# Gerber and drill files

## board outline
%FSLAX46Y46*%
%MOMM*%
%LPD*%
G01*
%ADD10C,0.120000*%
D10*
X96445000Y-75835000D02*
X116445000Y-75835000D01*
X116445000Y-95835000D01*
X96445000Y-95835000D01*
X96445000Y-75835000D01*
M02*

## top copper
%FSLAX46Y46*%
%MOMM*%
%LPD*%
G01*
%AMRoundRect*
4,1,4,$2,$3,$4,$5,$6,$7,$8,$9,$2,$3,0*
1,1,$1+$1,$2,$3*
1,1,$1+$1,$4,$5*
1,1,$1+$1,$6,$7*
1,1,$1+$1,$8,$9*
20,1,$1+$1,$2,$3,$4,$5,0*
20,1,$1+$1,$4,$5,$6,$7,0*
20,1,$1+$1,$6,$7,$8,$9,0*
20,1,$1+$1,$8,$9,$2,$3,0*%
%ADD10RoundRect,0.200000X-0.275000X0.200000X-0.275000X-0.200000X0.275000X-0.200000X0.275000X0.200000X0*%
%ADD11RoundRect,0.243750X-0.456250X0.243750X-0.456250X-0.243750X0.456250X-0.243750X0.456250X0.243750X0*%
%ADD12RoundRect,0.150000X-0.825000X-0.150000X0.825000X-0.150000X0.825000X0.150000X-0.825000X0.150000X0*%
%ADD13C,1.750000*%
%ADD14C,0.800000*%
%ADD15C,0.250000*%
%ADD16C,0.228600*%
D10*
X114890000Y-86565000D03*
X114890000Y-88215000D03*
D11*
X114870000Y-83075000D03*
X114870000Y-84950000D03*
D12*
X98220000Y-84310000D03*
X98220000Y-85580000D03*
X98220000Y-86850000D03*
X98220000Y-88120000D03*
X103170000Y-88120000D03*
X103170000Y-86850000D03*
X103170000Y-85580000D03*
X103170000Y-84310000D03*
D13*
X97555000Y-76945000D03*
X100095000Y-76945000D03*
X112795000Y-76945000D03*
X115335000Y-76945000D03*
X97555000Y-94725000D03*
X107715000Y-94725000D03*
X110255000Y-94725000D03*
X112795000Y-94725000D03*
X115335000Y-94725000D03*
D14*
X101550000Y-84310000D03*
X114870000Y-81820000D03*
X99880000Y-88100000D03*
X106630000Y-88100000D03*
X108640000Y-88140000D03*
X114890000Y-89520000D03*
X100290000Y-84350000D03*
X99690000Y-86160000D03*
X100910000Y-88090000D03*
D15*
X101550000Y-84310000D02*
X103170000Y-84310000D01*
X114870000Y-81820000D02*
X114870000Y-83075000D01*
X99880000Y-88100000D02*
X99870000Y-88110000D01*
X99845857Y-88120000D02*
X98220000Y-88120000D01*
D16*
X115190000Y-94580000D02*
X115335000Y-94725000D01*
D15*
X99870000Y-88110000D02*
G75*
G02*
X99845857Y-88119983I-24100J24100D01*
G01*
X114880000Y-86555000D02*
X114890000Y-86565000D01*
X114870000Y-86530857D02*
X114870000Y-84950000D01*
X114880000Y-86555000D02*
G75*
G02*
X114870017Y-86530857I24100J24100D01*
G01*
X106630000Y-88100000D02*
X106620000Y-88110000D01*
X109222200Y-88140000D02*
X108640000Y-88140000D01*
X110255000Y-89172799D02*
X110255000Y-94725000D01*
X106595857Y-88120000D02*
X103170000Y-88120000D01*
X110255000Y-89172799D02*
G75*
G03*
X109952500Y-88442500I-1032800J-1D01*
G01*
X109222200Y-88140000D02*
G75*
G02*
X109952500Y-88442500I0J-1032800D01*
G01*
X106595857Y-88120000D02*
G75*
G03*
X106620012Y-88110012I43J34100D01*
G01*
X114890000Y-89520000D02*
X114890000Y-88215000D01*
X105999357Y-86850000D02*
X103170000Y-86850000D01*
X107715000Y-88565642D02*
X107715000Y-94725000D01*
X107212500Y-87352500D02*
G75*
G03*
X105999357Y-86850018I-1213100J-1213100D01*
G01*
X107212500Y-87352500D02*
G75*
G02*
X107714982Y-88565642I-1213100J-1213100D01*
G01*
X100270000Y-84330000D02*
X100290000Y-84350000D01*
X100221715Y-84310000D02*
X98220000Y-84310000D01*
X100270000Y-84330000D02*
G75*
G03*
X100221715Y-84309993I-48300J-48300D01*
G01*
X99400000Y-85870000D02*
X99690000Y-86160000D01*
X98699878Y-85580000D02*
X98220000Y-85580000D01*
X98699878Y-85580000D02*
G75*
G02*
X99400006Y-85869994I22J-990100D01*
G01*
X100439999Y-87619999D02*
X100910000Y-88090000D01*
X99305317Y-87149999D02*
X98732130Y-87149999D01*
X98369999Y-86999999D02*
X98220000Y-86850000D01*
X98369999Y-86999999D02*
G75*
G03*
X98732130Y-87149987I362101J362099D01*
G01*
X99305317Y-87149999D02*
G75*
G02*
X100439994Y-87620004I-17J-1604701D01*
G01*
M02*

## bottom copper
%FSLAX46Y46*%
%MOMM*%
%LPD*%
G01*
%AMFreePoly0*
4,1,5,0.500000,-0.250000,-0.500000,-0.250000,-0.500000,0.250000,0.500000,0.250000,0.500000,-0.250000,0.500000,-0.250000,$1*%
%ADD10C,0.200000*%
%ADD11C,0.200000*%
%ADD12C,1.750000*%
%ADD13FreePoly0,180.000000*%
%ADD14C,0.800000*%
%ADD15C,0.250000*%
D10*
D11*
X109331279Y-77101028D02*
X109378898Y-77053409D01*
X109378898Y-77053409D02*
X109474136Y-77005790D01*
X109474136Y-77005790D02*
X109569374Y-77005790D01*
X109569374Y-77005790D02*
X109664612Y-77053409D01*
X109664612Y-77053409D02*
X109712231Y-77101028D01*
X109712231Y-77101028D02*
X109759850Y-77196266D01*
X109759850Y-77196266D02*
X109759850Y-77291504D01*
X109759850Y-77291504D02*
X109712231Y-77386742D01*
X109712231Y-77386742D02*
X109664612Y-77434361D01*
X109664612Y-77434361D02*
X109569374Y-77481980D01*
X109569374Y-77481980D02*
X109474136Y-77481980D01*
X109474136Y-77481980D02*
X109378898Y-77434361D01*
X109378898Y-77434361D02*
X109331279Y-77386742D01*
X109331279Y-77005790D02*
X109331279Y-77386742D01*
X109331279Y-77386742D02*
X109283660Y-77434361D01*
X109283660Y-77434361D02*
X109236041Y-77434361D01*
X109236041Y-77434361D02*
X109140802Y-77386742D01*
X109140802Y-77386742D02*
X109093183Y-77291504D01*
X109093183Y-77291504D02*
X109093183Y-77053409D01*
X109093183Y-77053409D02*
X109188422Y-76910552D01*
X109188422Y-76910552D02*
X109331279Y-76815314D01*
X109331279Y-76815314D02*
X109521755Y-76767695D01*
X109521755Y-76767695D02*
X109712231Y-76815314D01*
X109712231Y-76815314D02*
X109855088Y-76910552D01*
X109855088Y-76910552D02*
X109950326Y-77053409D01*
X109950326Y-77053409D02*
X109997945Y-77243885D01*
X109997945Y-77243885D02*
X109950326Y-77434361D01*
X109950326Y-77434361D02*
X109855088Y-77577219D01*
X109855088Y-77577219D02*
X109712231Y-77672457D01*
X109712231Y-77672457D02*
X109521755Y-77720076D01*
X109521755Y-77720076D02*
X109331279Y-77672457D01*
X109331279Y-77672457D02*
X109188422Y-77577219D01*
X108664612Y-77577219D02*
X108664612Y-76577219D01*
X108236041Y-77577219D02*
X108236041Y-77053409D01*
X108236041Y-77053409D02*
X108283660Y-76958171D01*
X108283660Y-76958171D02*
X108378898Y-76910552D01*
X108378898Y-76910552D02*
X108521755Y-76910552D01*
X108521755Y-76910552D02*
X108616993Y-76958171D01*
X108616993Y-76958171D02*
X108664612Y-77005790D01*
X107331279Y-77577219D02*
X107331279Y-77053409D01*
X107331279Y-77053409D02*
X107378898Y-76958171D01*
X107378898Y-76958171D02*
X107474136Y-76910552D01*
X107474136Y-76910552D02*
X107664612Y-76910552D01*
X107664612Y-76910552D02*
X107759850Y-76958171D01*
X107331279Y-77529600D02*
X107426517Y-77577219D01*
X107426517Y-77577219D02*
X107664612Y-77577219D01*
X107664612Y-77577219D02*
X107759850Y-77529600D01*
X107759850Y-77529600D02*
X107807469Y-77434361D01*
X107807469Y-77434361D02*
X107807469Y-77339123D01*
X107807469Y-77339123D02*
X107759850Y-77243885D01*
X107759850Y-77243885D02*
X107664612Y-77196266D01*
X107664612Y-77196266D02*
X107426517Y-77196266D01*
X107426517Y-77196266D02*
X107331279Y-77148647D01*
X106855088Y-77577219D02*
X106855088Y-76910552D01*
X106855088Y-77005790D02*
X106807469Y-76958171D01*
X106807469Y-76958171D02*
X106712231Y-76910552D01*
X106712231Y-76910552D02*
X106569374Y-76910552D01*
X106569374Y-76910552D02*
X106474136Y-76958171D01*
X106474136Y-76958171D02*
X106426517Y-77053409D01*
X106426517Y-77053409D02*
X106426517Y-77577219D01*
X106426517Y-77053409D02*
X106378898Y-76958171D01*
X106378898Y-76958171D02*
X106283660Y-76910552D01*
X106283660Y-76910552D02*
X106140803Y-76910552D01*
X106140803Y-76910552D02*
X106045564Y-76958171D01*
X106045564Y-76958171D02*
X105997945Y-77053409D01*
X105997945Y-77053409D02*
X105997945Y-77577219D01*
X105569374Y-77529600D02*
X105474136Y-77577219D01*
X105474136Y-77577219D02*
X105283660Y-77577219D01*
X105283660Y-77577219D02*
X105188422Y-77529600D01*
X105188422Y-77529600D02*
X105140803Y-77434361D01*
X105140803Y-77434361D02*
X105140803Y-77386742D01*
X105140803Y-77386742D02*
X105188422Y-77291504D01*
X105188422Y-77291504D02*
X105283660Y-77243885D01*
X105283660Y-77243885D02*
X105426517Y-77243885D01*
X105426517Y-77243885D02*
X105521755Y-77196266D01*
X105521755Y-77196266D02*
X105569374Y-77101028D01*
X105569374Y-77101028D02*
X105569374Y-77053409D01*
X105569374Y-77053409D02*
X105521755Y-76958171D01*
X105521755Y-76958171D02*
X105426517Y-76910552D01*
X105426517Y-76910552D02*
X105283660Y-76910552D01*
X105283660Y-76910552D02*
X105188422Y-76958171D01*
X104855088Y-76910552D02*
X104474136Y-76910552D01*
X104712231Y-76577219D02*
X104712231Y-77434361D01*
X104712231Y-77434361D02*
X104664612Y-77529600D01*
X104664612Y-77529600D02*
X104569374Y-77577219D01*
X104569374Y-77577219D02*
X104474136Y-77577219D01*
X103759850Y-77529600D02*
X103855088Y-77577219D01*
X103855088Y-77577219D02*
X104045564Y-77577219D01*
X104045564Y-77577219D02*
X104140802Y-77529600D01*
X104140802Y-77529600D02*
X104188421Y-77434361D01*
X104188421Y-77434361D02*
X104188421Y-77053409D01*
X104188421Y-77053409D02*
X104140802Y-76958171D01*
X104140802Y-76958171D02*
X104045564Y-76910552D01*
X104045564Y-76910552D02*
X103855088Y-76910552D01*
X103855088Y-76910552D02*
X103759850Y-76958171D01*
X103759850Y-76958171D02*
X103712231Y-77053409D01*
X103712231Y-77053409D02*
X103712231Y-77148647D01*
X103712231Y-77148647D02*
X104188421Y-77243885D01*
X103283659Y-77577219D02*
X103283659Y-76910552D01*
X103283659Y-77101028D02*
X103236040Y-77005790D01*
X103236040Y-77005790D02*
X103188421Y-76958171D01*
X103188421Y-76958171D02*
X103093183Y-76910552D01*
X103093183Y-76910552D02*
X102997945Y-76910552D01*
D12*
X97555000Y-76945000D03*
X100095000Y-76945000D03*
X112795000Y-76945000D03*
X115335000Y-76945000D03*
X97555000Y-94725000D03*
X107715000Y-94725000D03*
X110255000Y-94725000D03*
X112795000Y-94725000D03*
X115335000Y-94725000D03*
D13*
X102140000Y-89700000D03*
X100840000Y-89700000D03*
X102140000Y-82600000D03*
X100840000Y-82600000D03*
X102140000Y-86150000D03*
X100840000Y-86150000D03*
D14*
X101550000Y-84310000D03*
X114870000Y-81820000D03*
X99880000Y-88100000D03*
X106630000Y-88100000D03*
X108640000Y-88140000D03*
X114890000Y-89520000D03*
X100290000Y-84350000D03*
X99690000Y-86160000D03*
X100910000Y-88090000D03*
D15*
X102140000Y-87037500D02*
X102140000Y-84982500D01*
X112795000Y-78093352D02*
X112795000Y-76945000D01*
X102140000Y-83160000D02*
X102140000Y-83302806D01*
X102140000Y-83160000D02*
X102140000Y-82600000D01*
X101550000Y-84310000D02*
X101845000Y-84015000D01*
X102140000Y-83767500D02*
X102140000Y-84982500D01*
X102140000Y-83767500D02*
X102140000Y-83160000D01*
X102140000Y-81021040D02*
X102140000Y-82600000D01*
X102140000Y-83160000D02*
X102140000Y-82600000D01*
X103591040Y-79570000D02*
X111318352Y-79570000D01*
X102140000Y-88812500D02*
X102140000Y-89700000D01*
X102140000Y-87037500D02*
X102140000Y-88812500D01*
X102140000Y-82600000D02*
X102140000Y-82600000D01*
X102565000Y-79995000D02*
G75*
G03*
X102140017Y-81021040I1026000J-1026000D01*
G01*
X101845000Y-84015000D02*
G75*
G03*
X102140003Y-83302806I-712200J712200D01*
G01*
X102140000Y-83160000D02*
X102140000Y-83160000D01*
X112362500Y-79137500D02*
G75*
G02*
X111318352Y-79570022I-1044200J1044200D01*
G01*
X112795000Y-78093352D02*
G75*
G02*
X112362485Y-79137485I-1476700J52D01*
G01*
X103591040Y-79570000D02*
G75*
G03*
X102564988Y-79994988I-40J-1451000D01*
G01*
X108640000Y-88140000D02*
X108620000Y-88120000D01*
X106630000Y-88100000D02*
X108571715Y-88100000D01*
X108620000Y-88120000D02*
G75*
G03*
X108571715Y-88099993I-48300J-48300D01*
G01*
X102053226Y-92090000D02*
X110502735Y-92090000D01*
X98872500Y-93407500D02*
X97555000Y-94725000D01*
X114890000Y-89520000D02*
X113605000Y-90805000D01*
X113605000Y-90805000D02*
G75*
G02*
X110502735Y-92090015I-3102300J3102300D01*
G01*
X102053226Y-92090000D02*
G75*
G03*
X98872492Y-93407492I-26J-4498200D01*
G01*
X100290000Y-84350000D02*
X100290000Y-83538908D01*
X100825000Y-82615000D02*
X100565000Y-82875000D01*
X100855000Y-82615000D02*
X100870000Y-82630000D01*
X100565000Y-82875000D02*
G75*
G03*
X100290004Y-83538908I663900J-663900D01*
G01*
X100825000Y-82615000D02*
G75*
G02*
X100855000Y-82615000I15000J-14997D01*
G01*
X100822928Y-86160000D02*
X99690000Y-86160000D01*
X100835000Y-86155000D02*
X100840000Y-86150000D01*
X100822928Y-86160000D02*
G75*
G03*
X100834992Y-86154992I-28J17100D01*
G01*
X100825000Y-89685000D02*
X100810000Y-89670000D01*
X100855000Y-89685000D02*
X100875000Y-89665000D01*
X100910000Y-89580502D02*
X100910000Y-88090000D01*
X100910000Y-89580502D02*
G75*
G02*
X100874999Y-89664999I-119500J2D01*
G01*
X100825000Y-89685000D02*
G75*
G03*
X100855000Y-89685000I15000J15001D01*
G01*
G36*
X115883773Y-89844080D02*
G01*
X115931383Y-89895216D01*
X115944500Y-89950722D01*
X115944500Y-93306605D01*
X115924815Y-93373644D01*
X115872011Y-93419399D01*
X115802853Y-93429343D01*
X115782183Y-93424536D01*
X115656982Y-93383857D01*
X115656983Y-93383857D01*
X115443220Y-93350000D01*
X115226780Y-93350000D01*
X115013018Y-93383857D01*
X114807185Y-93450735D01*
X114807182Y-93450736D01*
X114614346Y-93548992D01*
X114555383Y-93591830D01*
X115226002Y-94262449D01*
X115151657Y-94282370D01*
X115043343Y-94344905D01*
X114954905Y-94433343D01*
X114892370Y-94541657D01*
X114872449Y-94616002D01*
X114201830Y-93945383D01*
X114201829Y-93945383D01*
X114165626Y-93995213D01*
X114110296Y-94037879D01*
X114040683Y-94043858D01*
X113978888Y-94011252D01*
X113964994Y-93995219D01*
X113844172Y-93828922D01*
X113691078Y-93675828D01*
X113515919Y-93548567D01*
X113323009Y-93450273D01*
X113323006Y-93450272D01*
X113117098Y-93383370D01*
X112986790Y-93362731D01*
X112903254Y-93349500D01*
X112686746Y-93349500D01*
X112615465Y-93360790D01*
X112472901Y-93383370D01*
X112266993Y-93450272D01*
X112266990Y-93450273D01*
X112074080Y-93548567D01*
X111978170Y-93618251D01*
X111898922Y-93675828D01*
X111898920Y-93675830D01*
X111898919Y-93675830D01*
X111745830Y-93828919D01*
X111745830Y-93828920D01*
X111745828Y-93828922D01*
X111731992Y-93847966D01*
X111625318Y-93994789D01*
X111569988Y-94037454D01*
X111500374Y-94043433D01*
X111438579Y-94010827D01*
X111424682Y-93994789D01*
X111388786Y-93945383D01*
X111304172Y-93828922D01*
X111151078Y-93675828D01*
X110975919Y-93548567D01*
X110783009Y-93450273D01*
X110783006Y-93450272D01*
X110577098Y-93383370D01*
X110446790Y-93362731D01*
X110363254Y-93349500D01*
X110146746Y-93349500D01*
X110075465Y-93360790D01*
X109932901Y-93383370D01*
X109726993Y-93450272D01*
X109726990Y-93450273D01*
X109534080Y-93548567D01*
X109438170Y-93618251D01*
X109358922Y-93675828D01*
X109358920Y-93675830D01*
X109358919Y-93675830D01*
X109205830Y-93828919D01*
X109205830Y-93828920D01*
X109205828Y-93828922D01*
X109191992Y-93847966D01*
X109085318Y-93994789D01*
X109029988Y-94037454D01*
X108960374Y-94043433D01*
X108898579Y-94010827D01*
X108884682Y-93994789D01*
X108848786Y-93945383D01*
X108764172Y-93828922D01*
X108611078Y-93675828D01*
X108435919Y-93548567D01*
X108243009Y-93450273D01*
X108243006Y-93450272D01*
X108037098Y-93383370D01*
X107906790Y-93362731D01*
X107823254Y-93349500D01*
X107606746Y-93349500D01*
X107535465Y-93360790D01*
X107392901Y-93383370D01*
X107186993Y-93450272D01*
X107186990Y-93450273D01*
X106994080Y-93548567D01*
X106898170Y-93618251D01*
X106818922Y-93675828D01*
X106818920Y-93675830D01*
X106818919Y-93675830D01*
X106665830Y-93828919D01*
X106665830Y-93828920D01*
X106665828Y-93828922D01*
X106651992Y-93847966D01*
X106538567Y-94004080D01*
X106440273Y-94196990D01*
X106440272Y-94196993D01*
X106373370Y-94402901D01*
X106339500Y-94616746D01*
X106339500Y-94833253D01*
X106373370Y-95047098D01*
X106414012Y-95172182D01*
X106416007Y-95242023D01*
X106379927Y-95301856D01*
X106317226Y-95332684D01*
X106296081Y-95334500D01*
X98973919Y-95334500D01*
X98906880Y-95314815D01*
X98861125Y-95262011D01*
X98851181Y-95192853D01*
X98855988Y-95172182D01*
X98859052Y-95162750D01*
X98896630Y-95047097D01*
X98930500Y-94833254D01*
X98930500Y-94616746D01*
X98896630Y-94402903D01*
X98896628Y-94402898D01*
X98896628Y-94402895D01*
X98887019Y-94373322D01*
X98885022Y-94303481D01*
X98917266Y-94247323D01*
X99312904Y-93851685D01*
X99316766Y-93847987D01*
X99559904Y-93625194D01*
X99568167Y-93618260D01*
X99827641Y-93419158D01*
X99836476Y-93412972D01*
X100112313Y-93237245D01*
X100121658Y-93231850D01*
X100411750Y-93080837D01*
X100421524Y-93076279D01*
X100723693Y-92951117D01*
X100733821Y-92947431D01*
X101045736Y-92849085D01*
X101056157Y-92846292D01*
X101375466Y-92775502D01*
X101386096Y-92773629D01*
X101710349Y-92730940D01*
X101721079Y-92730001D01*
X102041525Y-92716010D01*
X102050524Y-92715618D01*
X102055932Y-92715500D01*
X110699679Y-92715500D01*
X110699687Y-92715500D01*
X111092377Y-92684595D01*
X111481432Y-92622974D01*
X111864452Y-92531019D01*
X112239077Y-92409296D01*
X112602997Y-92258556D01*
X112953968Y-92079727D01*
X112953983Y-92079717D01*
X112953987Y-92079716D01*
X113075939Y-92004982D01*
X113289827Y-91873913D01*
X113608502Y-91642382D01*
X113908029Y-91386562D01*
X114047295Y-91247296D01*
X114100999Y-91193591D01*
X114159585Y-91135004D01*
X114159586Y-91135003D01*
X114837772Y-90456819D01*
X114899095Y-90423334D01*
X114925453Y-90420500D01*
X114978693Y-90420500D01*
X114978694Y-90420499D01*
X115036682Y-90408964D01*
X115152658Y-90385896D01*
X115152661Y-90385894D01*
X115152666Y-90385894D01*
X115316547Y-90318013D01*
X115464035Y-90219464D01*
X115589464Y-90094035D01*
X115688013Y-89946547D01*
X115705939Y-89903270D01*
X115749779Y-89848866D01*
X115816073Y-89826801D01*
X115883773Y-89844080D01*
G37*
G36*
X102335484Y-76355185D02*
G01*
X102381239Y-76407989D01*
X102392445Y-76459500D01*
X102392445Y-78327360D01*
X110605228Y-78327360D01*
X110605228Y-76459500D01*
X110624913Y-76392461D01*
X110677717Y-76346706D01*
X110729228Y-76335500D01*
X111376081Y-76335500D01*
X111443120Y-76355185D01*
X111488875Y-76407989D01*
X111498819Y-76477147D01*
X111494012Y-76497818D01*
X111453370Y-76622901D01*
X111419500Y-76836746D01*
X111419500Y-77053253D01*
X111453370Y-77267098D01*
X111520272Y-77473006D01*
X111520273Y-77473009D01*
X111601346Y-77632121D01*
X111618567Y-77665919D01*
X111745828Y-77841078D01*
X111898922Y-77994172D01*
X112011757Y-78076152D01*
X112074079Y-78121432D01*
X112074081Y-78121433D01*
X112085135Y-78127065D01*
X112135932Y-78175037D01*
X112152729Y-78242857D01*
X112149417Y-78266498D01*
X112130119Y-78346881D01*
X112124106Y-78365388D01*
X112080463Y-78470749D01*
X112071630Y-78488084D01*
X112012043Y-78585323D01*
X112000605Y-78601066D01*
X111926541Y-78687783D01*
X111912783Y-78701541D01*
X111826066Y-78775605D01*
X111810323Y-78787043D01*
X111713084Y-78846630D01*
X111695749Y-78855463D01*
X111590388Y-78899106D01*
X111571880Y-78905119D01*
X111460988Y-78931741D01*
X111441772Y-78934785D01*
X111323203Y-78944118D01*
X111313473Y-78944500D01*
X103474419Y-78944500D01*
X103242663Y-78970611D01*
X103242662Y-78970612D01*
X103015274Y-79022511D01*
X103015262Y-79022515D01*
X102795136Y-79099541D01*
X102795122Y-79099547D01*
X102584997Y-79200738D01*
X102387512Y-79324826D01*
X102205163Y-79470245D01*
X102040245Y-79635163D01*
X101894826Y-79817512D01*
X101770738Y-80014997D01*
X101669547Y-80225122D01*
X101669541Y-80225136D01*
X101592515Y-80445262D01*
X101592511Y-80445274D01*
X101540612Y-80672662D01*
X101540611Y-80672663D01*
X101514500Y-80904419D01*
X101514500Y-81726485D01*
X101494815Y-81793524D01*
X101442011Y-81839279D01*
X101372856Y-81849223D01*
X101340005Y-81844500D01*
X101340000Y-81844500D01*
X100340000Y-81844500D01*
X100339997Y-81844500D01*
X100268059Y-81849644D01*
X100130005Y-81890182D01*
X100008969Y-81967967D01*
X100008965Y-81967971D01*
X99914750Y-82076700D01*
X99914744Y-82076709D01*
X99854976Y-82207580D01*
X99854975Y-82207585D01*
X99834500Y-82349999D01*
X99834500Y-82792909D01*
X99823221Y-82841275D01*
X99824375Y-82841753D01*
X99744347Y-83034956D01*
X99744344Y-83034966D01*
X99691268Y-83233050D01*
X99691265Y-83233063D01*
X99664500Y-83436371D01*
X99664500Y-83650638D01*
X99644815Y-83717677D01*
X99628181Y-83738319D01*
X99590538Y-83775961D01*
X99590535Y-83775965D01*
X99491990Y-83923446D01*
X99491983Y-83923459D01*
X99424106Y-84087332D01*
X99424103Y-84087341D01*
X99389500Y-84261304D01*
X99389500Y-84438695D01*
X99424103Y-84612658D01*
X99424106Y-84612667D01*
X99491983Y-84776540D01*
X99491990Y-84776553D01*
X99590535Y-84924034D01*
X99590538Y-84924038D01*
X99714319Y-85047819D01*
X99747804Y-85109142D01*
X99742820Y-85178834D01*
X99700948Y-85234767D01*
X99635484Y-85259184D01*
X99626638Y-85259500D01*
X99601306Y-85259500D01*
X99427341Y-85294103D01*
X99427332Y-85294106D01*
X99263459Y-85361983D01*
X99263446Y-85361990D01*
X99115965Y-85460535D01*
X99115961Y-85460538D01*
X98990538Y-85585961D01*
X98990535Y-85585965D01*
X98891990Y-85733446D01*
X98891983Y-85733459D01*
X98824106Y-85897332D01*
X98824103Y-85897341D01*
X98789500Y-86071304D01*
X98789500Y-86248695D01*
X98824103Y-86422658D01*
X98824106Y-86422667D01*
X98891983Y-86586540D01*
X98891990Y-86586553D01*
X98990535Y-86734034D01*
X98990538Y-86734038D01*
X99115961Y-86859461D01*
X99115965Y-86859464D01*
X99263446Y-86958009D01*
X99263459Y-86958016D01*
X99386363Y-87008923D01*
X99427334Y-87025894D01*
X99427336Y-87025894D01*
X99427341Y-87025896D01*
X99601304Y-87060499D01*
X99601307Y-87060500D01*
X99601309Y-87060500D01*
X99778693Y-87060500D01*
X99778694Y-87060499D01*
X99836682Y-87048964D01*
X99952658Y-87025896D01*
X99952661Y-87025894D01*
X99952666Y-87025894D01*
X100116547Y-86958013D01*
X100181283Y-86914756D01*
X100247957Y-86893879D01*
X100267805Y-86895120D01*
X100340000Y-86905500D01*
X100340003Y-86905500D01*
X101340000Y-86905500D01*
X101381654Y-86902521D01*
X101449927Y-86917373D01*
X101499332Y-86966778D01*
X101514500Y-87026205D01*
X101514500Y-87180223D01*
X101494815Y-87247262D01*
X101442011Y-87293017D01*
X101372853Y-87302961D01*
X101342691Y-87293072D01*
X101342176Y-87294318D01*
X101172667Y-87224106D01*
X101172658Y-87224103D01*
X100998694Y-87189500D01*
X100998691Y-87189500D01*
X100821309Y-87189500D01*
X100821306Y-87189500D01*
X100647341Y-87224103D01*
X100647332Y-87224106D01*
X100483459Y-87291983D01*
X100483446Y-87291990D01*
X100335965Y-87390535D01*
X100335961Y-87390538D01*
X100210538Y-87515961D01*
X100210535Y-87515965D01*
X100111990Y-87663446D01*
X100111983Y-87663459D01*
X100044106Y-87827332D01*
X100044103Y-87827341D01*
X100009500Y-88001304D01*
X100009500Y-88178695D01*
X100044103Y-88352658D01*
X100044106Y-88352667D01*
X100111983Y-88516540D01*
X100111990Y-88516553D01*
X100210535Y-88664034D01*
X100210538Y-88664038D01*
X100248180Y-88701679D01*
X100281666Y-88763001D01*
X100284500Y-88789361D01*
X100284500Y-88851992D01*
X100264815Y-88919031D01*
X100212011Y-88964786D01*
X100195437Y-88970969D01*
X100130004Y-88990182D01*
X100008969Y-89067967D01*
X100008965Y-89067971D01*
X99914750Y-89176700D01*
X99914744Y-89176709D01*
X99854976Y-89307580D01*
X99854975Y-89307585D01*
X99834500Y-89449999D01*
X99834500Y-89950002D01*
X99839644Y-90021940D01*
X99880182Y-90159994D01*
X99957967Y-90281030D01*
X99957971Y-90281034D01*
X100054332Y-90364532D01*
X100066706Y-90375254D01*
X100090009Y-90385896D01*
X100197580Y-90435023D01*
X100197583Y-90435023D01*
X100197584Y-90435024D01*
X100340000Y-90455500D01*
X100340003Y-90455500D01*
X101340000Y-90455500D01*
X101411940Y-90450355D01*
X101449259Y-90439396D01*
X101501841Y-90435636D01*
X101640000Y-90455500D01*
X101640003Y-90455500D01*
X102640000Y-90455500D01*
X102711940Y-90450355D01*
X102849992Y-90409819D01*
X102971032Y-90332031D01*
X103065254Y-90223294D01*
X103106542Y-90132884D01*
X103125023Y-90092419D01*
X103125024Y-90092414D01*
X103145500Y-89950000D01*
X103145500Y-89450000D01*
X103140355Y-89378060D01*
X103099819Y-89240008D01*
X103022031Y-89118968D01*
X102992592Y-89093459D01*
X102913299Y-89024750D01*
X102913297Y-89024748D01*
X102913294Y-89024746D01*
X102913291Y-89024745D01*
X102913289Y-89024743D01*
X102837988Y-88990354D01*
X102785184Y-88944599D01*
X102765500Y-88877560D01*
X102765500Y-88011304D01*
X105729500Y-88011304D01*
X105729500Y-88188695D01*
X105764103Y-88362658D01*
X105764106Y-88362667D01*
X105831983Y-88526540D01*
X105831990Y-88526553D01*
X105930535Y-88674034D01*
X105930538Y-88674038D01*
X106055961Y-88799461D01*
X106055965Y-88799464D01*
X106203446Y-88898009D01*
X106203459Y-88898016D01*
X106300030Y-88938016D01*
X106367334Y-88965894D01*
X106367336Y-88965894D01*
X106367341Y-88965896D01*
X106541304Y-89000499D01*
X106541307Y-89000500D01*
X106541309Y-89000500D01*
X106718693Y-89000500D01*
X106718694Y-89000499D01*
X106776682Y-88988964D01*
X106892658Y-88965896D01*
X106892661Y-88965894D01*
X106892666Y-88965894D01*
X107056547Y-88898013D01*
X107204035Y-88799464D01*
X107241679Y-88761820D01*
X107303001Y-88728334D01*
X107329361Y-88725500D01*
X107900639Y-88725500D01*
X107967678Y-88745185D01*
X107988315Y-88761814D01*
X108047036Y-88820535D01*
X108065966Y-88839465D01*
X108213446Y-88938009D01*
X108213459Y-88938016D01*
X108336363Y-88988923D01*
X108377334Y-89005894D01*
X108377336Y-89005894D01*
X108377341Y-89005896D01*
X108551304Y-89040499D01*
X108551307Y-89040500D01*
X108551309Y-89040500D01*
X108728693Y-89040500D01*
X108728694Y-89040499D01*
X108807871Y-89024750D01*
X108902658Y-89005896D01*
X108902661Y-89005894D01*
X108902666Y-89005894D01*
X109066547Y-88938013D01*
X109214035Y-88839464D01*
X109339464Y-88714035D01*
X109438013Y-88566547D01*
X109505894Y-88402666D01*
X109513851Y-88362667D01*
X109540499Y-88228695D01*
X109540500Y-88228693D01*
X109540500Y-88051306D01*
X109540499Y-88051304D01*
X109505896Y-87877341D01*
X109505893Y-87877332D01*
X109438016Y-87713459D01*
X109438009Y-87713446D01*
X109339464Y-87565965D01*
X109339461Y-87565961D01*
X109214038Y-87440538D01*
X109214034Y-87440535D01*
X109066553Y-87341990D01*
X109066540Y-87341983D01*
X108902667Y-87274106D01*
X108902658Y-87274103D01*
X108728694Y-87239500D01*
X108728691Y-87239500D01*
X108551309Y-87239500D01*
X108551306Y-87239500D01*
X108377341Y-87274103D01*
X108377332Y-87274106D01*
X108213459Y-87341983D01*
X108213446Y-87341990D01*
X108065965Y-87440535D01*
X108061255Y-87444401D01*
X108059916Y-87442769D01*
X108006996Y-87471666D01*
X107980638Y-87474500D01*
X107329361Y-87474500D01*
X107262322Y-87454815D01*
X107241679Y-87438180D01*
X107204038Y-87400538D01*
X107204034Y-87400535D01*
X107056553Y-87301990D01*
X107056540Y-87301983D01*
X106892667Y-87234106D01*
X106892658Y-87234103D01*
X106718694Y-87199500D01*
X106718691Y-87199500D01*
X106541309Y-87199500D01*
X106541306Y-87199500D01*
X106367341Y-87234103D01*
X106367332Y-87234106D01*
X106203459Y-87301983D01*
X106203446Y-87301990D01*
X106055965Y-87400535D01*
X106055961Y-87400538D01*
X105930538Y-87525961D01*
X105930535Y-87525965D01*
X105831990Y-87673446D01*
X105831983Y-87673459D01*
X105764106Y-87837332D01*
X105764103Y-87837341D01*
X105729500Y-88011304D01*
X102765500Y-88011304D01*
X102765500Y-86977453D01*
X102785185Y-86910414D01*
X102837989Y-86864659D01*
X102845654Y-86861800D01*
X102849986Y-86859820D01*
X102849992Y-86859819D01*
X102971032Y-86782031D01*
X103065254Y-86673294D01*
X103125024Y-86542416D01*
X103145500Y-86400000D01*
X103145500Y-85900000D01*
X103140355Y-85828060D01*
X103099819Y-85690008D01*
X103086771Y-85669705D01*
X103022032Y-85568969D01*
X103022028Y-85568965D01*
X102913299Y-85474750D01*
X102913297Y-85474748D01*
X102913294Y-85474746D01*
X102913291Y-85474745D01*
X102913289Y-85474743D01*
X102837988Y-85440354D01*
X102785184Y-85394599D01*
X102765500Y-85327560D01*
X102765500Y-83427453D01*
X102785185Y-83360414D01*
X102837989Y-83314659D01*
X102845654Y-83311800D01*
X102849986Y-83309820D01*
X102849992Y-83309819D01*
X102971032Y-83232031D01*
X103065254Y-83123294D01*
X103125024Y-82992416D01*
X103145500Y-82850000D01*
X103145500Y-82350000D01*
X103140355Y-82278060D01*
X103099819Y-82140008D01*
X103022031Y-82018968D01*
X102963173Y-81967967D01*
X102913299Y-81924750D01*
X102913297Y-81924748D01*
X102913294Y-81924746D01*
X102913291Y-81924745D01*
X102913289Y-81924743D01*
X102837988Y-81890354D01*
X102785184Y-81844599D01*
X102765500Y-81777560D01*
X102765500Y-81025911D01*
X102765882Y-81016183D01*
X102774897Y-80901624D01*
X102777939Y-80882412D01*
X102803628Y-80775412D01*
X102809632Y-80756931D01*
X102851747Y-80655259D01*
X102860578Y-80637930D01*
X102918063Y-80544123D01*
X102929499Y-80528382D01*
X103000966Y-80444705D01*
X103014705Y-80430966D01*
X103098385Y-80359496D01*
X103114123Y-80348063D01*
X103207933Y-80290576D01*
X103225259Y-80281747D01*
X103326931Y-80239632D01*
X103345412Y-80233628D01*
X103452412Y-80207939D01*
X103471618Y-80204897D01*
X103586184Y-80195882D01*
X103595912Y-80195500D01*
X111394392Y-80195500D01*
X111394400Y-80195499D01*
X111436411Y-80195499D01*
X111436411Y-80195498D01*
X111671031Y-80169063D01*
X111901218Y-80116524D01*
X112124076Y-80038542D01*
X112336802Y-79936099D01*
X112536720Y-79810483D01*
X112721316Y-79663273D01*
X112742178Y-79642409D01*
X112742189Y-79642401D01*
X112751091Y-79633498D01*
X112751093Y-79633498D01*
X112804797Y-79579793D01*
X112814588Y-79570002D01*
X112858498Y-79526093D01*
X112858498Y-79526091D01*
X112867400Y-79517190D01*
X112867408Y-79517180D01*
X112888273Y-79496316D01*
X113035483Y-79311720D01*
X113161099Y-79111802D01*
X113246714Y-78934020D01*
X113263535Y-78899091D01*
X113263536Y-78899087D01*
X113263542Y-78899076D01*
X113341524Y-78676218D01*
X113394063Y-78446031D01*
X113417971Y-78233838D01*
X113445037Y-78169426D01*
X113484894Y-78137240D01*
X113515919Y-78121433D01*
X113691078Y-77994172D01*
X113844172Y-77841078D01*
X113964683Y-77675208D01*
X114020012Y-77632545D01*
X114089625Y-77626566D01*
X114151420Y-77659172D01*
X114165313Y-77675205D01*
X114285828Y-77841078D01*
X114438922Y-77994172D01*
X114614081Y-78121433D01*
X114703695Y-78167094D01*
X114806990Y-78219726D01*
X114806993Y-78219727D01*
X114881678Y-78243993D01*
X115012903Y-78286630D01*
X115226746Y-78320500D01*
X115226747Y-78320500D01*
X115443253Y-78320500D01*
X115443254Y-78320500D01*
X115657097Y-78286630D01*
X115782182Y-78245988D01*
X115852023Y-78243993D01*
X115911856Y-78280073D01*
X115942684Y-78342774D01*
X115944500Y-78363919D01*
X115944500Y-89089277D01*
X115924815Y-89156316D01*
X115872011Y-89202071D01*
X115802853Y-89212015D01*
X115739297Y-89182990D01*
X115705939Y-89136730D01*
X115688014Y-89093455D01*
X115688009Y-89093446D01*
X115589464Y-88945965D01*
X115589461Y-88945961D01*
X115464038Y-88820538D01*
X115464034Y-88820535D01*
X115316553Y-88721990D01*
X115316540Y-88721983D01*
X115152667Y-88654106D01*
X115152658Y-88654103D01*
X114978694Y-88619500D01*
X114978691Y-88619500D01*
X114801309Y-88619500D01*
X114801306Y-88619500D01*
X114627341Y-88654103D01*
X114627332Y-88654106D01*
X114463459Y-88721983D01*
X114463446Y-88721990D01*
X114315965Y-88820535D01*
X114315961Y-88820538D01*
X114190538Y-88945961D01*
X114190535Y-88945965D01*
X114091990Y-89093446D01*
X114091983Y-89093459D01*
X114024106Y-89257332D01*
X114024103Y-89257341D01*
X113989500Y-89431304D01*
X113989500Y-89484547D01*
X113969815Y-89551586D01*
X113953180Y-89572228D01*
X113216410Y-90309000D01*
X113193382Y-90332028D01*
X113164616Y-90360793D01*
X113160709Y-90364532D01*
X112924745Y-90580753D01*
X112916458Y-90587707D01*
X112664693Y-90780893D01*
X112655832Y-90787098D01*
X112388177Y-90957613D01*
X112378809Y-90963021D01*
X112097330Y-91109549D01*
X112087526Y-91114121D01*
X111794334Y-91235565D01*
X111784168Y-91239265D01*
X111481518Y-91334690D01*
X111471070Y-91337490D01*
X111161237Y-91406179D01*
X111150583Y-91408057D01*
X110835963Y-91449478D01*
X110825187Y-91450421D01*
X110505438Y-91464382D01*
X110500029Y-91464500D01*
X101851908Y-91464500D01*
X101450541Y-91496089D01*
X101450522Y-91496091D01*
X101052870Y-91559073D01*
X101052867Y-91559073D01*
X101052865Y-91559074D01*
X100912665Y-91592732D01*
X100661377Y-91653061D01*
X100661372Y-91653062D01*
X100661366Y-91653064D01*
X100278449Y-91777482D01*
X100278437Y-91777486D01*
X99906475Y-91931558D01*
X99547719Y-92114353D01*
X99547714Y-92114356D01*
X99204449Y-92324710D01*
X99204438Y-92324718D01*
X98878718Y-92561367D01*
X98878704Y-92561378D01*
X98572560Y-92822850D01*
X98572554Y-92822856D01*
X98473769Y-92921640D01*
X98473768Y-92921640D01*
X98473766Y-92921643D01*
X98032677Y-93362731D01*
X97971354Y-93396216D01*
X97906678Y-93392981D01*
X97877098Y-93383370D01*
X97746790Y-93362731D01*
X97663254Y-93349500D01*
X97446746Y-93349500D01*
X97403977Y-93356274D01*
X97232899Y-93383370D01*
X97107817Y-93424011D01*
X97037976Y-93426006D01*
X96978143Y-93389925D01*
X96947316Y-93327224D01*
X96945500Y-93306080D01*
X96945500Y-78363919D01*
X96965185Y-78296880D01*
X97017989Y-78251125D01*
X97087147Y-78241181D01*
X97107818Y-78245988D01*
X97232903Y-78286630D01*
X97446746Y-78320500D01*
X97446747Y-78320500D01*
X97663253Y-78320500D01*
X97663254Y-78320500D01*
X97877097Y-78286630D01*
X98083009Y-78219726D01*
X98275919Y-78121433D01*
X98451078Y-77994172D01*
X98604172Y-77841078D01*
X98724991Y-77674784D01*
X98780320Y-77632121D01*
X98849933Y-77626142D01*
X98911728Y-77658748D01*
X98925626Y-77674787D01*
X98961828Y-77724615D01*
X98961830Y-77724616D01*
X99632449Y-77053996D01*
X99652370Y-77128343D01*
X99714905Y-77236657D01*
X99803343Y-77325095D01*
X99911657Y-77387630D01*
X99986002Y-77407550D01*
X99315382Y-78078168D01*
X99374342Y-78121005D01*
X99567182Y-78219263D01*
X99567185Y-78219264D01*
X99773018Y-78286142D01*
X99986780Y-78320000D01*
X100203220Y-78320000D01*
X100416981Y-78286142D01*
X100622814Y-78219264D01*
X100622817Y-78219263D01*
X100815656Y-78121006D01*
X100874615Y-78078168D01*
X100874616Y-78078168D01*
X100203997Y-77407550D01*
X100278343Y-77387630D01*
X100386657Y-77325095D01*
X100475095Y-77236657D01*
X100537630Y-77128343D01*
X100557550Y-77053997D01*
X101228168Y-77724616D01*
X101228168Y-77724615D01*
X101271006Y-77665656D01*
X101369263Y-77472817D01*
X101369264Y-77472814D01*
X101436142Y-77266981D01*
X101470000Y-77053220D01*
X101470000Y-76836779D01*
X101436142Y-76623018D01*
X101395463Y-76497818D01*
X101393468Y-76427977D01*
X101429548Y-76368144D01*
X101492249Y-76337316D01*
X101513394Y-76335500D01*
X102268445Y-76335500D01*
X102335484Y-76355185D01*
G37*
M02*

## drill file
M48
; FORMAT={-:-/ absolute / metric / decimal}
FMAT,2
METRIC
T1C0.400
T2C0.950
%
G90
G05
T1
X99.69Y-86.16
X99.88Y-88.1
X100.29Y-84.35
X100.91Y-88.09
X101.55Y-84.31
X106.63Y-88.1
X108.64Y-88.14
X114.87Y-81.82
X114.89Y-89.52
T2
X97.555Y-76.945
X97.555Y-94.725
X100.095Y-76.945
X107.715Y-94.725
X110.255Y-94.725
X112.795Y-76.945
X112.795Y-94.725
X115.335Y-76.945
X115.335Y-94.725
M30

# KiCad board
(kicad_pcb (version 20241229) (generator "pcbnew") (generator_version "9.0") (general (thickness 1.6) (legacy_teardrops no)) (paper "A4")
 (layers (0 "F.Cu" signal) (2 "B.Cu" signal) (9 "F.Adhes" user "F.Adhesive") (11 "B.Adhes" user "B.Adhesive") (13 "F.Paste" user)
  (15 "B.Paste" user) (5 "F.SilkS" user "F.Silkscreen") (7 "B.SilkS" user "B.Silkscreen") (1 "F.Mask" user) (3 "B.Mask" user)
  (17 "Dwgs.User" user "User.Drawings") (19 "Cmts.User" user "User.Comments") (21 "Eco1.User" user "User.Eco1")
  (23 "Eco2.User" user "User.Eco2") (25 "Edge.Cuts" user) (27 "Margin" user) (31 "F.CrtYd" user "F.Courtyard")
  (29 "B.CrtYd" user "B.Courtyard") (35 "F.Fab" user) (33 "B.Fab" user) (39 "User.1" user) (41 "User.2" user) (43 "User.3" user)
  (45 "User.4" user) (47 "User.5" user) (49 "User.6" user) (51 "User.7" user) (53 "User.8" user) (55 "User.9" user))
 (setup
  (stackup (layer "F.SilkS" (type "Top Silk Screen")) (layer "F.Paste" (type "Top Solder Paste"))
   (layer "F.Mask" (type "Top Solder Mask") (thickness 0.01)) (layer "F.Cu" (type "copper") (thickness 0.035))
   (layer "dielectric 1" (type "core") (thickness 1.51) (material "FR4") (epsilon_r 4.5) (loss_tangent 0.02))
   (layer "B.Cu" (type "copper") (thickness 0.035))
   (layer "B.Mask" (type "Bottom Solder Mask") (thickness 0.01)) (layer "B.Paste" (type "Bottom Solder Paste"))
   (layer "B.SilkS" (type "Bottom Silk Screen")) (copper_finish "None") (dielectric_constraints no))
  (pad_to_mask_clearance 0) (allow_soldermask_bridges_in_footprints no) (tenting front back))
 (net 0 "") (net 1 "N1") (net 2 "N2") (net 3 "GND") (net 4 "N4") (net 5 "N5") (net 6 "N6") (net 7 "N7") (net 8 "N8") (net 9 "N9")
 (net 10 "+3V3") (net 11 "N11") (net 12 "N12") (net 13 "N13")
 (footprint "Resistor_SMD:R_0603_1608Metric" (layer "F.Cu") (at 114.89 87.39 -90)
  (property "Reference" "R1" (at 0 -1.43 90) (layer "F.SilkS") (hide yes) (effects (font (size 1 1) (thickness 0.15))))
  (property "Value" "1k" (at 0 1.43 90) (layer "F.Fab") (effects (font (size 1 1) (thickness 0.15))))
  (pad "1" smd roundrect (at -0.825 0 270) (size 0.8 0.95) (layers "F.Cu" "F.Mask" "F.Paste") (roundrect_rratio 0.25) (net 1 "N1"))
  (pad "2" smd roundrect (at 0.825 0 270) (size 0.8 0.95) (layers "F.Cu" "F.Mask" "F.Paste") (roundrect_rratio 0.25) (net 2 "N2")))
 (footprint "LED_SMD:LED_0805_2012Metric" (layer "F.Cu") (at 114.87 84.0125 -90)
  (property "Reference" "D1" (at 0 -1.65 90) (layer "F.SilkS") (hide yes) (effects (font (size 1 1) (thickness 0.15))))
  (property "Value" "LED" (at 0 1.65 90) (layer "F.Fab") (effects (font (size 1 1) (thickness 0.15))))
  (pad "1" smd roundrect (at -0.9375 0 270) (size 0.975 1.4) (layers "F.Cu" "F.Mask" "F.Paste") (roundrect_rratio 0.25) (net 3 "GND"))
  (pad "2" smd roundrect (at 0.9375 0 270) (size 0.975 1.4) (layers "F.Cu" "F.Mask" "F.Paste") (roundrect_rratio 0.25) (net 1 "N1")))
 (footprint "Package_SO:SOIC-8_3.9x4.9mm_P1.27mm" (layer "F.Cu") (at 100.695 86.215)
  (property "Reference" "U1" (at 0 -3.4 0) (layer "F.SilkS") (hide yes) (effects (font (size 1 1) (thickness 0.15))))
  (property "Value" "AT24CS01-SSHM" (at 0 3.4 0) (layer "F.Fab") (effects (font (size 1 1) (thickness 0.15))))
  (pad "1" smd roundrect (at -2.475 -1.905) (size 1.95 0.6) (layers "F.Cu" "F.Mask" "F.Paste") (roundrect_rratio 0.25) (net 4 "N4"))
  (pad "2" smd roundrect (at -2.475 -0.635) (size 1.95 0.6) (layers "F.Cu" "F.Mask" "F.Paste") (roundrect_rratio 0.25) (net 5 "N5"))
  (pad "3" smd roundrect (at -2.475 0.635) (size 1.95 0.6) (layers "F.Cu" "F.Mask" "F.Paste") (roundrect_rratio 0.25) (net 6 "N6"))
  (pad "4" smd roundrect (at -2.475 1.905) (size 1.95 0.6) (layers "F.Cu" "F.Mask" "F.Paste") (roundrect_rratio 0.25) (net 3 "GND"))
  (pad "5" smd roundrect (at 2.475 1.905) (size 1.95 0.6) (layers "F.Cu" "F.Mask" "F.Paste") (roundrect_rratio 0.25) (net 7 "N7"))
  (pad "6" smd roundrect (at 2.475 0.635) (size 1.95 0.6) (layers "F.Cu" "F.Mask" "F.Paste") (roundrect_rratio 0.25) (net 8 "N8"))
  (pad "7" smd roundrect (at 2.475 -0.635) (size 1.95 0.6) (layers "F.Cu" "F.Mask" "F.Paste") (roundrect_rratio 0.25) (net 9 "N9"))
  (pad "8" smd roundrect (at 2.475 -1.905) (size 1.95 0.6) (layers "F.Cu" "F.Mask" "F.Paste") (roundrect_rratio 0.25) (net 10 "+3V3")))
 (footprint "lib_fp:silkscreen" (layer "F.Cu") (at 106.5 85.79)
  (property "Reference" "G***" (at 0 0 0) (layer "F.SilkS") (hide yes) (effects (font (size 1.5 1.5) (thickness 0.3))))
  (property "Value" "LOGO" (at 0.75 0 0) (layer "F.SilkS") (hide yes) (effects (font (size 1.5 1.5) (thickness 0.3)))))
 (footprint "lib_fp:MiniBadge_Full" (layer "F.Cu") (at 96.285 75.675)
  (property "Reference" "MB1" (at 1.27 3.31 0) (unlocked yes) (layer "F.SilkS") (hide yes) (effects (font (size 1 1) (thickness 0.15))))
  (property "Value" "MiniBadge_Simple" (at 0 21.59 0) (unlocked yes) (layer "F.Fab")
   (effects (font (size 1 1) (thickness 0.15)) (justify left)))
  (fp_rect (start 20.16 20.16) (end 0.16 0.16) (stroke (width 0.12) (type solid)) (fill no) (layer "Edge.Cuts"))
  (pad "1" thru_hole circle (at 1.27 1.27) (size 1.75 1.75) (drill 0.95) (layers "*.Cu" "*.Mask") (remove_unused_layers no) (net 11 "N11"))
  (pad "2" thru_hole circle (at 3.81 1.27) (size 1.75 1.75) (drill 0.95) (layers "*.Cu" "*.Mask") (remove_unused_layers no) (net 3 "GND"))
  (pad "7" thru_hole circle (at 16.51 1.27) (size 1.75 1.75) (drill 0.95) (layers "*.Cu" "*.Mask") (remove_unused_layers no) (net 10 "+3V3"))
  (pad "8" thru_hole circle (at 19.05 1.27) (size 1.75 1.75) (drill 0.95) (layers "*.Cu" "*.Mask") (remove_unused_layers no) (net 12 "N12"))
  (pad "9" thru_hole circle (at 1.27 19.05) (size 1.75 1.75) (drill 0.95) (layers "*.Cu" "*.Mask") (remove_unused_layers no) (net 2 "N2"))
  (pad "13" thru_hole circle (at 11.43 19.05) (size 1.75 1.75) (drill 0.95) (layers "*.Cu" "*.Mask") (remove_unused_layers no) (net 8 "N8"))
  (pad "14" thru_hole circle (at 13.97 19.05) (size 1.75 1.75) (drill 0.95) (layers "*.Cu" "*.Mask") (remove_unused_layers no) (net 7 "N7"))
  (pad "15" thru_hole circle (at 16.51 19.05) (size 1.75 1.75) (drill 0.95) (layers "*.Cu" "*.Mask") (remove_unused_layers no)
   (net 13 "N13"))
  (pad "16" thru_hole circle (at 19.05 19.05) (size 1.75 1.75) (drill 0.95) (layers "*.Cu" "*.Mask") (remove_unused_layers no) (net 3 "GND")))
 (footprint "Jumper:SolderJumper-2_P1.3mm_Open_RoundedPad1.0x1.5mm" (layer "B.Cu") (at 101.49 89.7 180)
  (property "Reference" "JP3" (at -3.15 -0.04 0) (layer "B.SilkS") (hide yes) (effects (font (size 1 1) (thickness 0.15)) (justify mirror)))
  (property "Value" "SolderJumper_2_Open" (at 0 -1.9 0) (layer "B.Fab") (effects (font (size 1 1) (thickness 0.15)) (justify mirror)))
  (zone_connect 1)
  (pad "1" smd custom (at -0.65 0 180) (size 1 0.5) (layers "B.Cu" "B.Mask") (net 10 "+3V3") (zone_connect 2) (thermal_bridge_angle 45)
   (options (clearance outline) (anchor rect)) (primitives))
  (pad "2" smd custom (at 0.65 0 180) (size 1 0.5) (layers "B.Cu" "B.Mask") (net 6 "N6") (zone_connect 2) (thermal_bridge_angle 45)
   (options (clearance outline) (anchor rect)) (primitives)))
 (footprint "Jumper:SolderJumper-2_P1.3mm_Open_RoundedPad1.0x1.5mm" (layer "B.Cu") (at 101.49 82.6 180)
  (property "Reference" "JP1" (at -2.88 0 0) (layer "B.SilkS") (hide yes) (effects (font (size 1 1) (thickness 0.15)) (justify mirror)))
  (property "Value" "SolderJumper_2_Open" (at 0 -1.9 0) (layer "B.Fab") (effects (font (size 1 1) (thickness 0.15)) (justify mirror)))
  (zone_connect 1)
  (pad "1" smd custom (at -0.65 0 180) (size 1 0.5) (layers "B.Cu" "B.Mask") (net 10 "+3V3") (zone_connect 2) (thermal_bridge_angle 45)
   (options (clearance outline) (anchor rect)) (primitives))
  (pad "2" smd custom (at 0.65 0 180) (size 1 0.5) (layers "B.Cu" "B.Mask") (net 4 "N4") (zone_connect 2) (thermal_bridge_angle 45)
   (options (clearance outline) (anchor rect)) (primitives)))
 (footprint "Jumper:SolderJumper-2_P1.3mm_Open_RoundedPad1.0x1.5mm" (layer "B.Cu") (at 101.49 86.15 180)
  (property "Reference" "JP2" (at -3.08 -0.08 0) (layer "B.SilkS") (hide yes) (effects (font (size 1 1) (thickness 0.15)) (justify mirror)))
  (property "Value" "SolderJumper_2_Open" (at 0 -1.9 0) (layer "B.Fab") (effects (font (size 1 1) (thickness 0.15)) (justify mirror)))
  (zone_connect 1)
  (pad "1" smd custom (at -0.65 0 180) (size 1 0.5) (layers "B.Cu" "B.Mask") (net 10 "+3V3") (zone_connect 2) (thermal_bridge_angle 45)
   (options (clearance outline) (anchor rect)) (primitives))
  (pad "2" smd custom (at 0.65 0 180) (size 1 0.5) (layers "B.Cu" "B.Mask") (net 5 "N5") (zone_connect 2) (thermal_bridge_angle 45)
   (options (clearance outline) (anchor rect)) (primitives)))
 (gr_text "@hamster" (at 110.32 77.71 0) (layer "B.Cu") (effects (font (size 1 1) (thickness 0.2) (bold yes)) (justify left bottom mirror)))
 (segment (start 101.55 84.31) (end 103.17 84.31) (width 0.25) (layer "F.Cu") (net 10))
 (via (at 101.55 84.31) (size 0.8) (drill 0.4) (layers "F.Cu" "B.Cu") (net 10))
 (segment (start 102.14 87.0375) (end 102.14 84.9825) (width 0.25) (layer "B.Cu") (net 10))
 (segment (start 112.795 78.093352) (end 112.795 76.945) (width 0.25) (layer "B.Cu") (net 10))
 (segment (start 102.14 83.16) (end 102.14 83.302806) (width 0.25) (layer "B.Cu") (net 10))
 (segment (start 102.14 83.16) (end 102.14 82.6) (width 0.25) (layer "B.Cu") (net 10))
 (segment (start 101.55 84.31) (end 101.845 84.015) (width 0.25) (layer "B.Cu") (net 10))
 (segment (start 102.14 83.7675) (end 102.14 84.9825) (width 0.25) (layer "B.Cu") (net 10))
 (segment (start 102.14 83.7675) (end 102.14 83.16) (width 0.25) (layer "B.Cu") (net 10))
 (segment (start 102.14 81.02104) (end 102.14 82.6) (width 0.25) (layer "B.Cu") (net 10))
 (segment (start 102.14 83.16) (end 102.14 82.6) (width 0.25) (layer "B.Cu") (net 10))
 (segment (start 103.59104 79.57) (end 111.318352 79.57) (width 0.25) (layer "B.Cu") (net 10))
 (segment (start 102.14 88.8125) (end 102.14 89.7) (width 0.25) (layer "B.Cu") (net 10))
 (segment (start 102.14 87.0375) (end 102.14 88.8125) (width 0.25) (layer "B.Cu") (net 10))
 (arc (start 102.14 82.6) (mid 102.14 82.6) (end 102.14 82.6) (width 0.25) (layer "B.Cu") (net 10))
 (arc (start 102.565 79.995) (mid 102.250453 80.465751) (end 102.14 81.02104) (width 0.25) (layer "B.Cu") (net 10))
 (arc (start 101.845 84.015) (mid 102.063331 83.688242) (end 102.14 83.302806) (width 0.25) (layer "B.Cu") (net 10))
 (arc (start 102.14 83.16) (mid 102.14 83.16) (end 102.14 83.16) (width 0.25) (layer "B.Cu") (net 10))
 (arc (start 112.3625 79.1375) (mid 111.88344 79.457596) (end 111.318352 79.57) (width 0.25) (layer "B.Cu") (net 10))
 (arc (start 112.795 78.093352) (mid 112.682596 78.65844) (end 112.3625 79.1375) (width 0.25) (layer "B.Cu") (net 10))
 (arc (start 103.59104 79.57) (mid 103.035751 79.680453) (end 102.565 79.995) (width 0.25) (layer "B.Cu") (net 10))
 (segment (start 114.87 81.82) (end 114.87 83.075) (width 0.25) (layer "F.Cu") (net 3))
 (segment (start 99.88 88.1) (end 99.87 88.11) (width 0.25) (layer "F.Cu") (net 3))
 (segment (start 99.845857 88.12) (end 98.22 88.12) (width 0.25) (layer "F.Cu") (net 3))
 (segment (start 115.19 94.58) (end 115.335 94.725) (width 0.2286) (layer "F.Cu") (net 3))
 (via (at 114.87 81.82) (size 0.8) (drill 0.4) (layers "F.Cu" "B.Cu") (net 3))
 (via (at 99.88 88.1) (size 0.8) (drill 0.4) (layers "F.Cu" "B.Cu") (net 3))
 (arc (start 99.87 88.11) (mid 99.858923 88.117401) (end 99.845857 88.12) (width 0.25) (layer "F.Cu") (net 3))
 (segment (start 114.88 86.555) (end 114.89 86.565) (width 0.25) (layer "F.Cu") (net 1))
 (segment (start 114.87 86.530857) (end 114.87 84.95) (width 0.25) (layer "F.Cu") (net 1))
 (arc (start 114.88 86.555) (mid 114.872598 86.543923) (end 114.87 86.530857) (width 0.25) (layer "F.Cu") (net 1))
 (segment (start 106.63 88.1) (end 106.62 88.11) (width 0.25) (layer "F.Cu") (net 7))
 (segment (start 109.2222 88.14) (end 108.64 88.14) (width 0.25) (layer "F.Cu") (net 7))
 (segment (start 110.255 89.172799) (end 110.255 94.725) (width 0.25) (layer "F.Cu") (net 7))
 (segment (start 106.595857 88.12) (end 103.17 88.12) (width 0.25) (layer "F.Cu") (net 7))
 (via (at 106.63 88.1) (size 0.8) (drill 0.4) (layers "F.Cu" "B.Cu") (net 7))
 (via (at 108.64 88.14) (size 0.8) (drill 0.4) (layers "F.Cu" "B.Cu") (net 7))
 (arc (start 110.255 89.172799) (mid 110.176382 88.777564) (end 109.9525 88.4425) (width 0.25) (layer "F.Cu") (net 7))
 (arc (start 109.2222 88.14) (mid 109.617435 88.218617) (end 109.9525 88.4425) (width 0.25) (layer "F.Cu") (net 7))
 (arc (start 106.595857 88.12) (mid 106.608923 88.117401) (end 106.62 88.11) (width 0.25) (layer "F.Cu") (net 7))
 (segment (start 108.64 88.14) (end 108.62 88.12) (width 0.25) (layer "B.Cu") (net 7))
 (segment (start 106.63 88.1) (end 108.571715 88.1) (width 0.25) (layer "B.Cu") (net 7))
 (arc (start 108.62 88.12) (mid 108.597846 88.105197) (end 108.571715 88.1) (width 0.25) (layer "B.Cu") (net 7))
 (segment (start 114.89 89.52) (end 114.89 88.215) (width 0.25) (layer "F.Cu") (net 2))
 (via (at 114.89 89.52) (size 0.8) (drill 0.4) (layers "F.Cu" "B.Cu") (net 2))
 (segment (start 102.053226 92.09) (end 110.502735 92.09) (width 0.25) (layer "B.Cu") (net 2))
 (segment (start 98.8725 93.4075) (end 97.555 94.725) (width 0.25) (layer "B.Cu") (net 2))
 (segment (start 114.89 89.52) (end 113.605 90.805) (width 0.25) (layer "B.Cu") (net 2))
 (arc (start 113.605 90.805) (mid 112.181668 91.756039) (end 110.502735 92.09) (width 0.25) (layer "B.Cu") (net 2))
 (arc (start 102.053226 92.09) (mid 100.331829 92.432407) (end 98.8725 93.4075) (width 0.25) (layer "B.Cu") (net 2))
 (segment (start 105.999357 86.85) (end 103.17 86.85) (width 0.25) (layer "F.Cu") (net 8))
 (segment (start 107.715 88.565642) (end 107.715 94.725) (width 0.25) (layer "F.Cu") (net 8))
 (arc (start 107.2125 87.3525) (mid 106.655905 86.980595) (end 105.999357 86.85) (width 0.25) (layer "F.Cu") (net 8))
 (arc (start 107.2125 87.3525) (mid 107.584404 87.909094) (end 107.715 88.565642) (width 0.25) (layer "F.Cu") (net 8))
 (segment (start 100.27 84.33) (end 100.29 84.35) (width 0.25) (layer "F.Cu") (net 4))
 (segment (start 100.221715 84.31) (end 98.22 84.31) (width 0.25) (layer "F.Cu") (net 4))
 (via (at 100.29 84.35) (size 0.8) (drill 0.4) (layers "F.Cu" "B.Cu") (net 4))
 (arc (start 100.27 84.33) (mid 100.247846 84.315197) (end 100.221715 84.31) (width 0.25) (layer "F.Cu") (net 4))
 (segment (start 100.29 84.35) (end 100.29 83.538908) (width 0.25) (layer "B.Cu") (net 4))
 (segment (start 100.825 82.615) (end 100.565 82.875) (width 0.25) (layer "B.Cu") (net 4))
 (segment (start 100.855 82.615) (end 100.87 82.63) (width 0.25) (layer "B.Cu") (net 4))
 (arc (start 100.565 82.875) (mid 100.36147 83.179603) (end 100.29 83.538908) (width 0.25) (layer "B.Cu") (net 4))
 (arc (start 100.825 82.615) (mid 100.84 82.608786) (end 100.855 82.615) (width 0.25) (layer "B.Cu") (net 4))
 (segment (start 99.4 85.87) (end 99.69 86.16) (width 0.25) (layer "F.Cu") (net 5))
 (segment (start 98.699878 85.58) (end 98.22 85.58) (width 0.25) (layer "F.Cu") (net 5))
 (via (at 99.69 86.16) (size 0.8) (drill 0.4) (layers "F.Cu" "B.Cu") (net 5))
 (arc (start 98.699878 85.58) (mid 99.078781 85.655368) (end 99.4 85.87) (width 0.25) (layer "F.Cu") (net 5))
 (segment (start 100.822928 86.16) (end 99.69 86.16) (width 0.25) (layer "B.Cu") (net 5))
 (segment (start 100.835 86.155) (end 100.84 86.15) (width 0.25) (layer "B.Cu") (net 5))
 (arc (start 100.822928 86.16) (mid 100.829461 86.1587) (end 100.835 86.155) (width 0.25) (layer "B.Cu") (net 5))
 (segment (start 100.439999 87.619999) (end 100.91 88.09) (width 0.25) (layer "F.Cu") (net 6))
 (segment (start 99.305317 87.149999) (end 98.73213 87.149999) (width 0.25) (layer "F.Cu") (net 6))
 (segment (start 98.369999 86.999999) (end 98.22 86.85) (width 0.25) (layer "F.Cu") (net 6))
 (via (at 100.91 88.09) (size 0.8) (drill 0.4) (layers "F.Cu" "B.Cu") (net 6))
 (arc (start 98.369999 86.999999) (mid 98.536146 87.111015) (end 98.73213 87.149999) (width 0.25) (layer "F.Cu") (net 6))
 (arc (start 99.305317 87.149999) (mid 99.919402 87.272148) (end 100.439999 87.619999) (width 0.25) (layer "F.Cu") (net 6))
 (segment (start 100.825 89.685) (end 100.81 89.67) (width 0.25) (layer "B.Cu") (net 6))
 (segment (start 100.855 89.685) (end 100.875 89.665) (width 0.25) (layer "B.Cu") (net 6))
 (segment (start 100.91 89.580502) (end 100.91 88.09) (width 0.25) (layer "B.Cu") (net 6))
 (arc (start 100.91 89.580502) (mid 100.900903 89.626232) (end 100.875 89.665) (width 0.25) (layer "B.Cu") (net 6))
 (arc (start 100.825 89.685) (mid 100.84 89.691213) (end 100.855 89.685) (width 0.25) (layer "B.Cu") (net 6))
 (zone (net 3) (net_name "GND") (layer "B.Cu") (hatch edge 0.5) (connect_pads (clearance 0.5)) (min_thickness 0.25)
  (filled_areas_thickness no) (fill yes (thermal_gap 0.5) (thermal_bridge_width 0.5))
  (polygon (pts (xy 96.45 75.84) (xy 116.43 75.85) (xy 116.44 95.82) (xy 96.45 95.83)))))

